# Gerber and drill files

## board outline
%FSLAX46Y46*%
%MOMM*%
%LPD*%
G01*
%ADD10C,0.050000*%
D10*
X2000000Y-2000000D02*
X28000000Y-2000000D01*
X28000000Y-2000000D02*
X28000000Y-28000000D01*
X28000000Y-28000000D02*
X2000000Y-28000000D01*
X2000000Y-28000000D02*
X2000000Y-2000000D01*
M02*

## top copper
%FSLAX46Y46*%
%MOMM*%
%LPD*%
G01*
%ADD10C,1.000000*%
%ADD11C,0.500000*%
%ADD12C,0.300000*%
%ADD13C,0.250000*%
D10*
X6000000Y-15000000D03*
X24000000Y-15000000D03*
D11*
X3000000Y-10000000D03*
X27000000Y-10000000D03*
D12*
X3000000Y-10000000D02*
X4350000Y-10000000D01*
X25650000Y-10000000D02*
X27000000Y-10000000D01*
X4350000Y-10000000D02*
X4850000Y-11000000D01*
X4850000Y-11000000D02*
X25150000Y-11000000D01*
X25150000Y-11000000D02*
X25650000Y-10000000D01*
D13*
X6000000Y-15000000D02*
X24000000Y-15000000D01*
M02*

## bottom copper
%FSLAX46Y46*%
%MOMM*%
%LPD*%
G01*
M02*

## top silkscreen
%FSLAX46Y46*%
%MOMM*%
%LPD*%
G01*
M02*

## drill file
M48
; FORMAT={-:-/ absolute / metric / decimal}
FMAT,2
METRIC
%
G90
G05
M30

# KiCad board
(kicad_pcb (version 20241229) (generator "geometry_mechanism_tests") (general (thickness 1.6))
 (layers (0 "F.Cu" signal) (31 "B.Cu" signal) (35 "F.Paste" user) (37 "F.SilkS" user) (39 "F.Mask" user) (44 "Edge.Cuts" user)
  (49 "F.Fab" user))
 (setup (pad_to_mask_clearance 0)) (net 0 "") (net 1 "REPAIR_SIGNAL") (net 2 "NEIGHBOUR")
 (gr_line (start 2.000000 2.000000) (end 28.000000 2.000000) (stroke (width .05) (type default)) (layer "Edge.Cuts"))
 (gr_line (start 28.000000 2.000000) (end 28.000000 28.000000) (stroke (width .05) (type default)) (layer "Edge.Cuts"))
 (gr_line (start 28.000000 28.000000) (end 2.000000 28.000000) (stroke (width .05) (type default)) (layer "Edge.Cuts"))
 (gr_line (start 2.000000 28.000000) (end 2.000000 2.000000) (stroke (width .05) (type default)) (layer "Edge.Cuts"))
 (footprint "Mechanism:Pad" (layer "F.Cu") (at 6.000000 15.000000)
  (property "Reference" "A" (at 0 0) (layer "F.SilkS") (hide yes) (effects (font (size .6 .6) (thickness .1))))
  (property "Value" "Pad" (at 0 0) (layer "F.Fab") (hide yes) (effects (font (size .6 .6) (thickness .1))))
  (pad "1" smd circle (at 0 0 31.000000) (size 1 1) (layers "F.Cu" "F.Paste" "F.Mask") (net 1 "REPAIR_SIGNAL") (clearance 0)))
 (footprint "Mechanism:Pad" (layer "F.Cu") (at 24.000000 15.000000)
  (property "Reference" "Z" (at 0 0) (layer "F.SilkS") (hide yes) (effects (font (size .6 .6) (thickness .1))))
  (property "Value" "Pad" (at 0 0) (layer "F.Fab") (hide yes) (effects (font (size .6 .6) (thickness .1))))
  (pad "1" smd circle (at 0 0 31.000000) (size 1 1) (layers "F.Cu" "F.Paste" "F.Mask") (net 1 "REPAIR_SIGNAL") (clearance 0)))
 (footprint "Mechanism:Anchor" (layer "F.Cu") (at 3 10)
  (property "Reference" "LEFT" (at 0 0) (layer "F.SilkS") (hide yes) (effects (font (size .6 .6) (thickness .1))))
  (pad "1" smd circle (at 0 0) (size .5 .5) (layers "F.Cu" "F.Paste" "F.Mask") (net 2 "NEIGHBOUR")))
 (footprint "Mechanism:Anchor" (layer "F.Cu") (at 27 10)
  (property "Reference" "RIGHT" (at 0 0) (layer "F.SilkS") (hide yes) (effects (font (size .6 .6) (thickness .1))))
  (pad "1" smd circle (at 0 0) (size .5 .5) (layers "F.Cu" "F.Paste" "F.Mask") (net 2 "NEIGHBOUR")))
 (segment (start 3.0 10.0) (end 4.35 10.0) (width .3) (layer "F.Cu") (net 2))
 (segment (start 25.65 10.0) (end 27.0 10.0) (width .3) (layer "F.Cu") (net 2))
 (segment (start 4.35 10.0) (end 4.85 11) (width .3) (layer "F.Cu") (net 2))
 (segment (start 4.85 11) (end 25.15 11) (width .3) (layer "F.Cu") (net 2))
 (segment (start 25.15 11) (end 25.65 10.0) (width .3) (layer "F.Cu") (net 2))
 (segment (start 6 15) (end 24 15) (width .25) (layer "F.Cu") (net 1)))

